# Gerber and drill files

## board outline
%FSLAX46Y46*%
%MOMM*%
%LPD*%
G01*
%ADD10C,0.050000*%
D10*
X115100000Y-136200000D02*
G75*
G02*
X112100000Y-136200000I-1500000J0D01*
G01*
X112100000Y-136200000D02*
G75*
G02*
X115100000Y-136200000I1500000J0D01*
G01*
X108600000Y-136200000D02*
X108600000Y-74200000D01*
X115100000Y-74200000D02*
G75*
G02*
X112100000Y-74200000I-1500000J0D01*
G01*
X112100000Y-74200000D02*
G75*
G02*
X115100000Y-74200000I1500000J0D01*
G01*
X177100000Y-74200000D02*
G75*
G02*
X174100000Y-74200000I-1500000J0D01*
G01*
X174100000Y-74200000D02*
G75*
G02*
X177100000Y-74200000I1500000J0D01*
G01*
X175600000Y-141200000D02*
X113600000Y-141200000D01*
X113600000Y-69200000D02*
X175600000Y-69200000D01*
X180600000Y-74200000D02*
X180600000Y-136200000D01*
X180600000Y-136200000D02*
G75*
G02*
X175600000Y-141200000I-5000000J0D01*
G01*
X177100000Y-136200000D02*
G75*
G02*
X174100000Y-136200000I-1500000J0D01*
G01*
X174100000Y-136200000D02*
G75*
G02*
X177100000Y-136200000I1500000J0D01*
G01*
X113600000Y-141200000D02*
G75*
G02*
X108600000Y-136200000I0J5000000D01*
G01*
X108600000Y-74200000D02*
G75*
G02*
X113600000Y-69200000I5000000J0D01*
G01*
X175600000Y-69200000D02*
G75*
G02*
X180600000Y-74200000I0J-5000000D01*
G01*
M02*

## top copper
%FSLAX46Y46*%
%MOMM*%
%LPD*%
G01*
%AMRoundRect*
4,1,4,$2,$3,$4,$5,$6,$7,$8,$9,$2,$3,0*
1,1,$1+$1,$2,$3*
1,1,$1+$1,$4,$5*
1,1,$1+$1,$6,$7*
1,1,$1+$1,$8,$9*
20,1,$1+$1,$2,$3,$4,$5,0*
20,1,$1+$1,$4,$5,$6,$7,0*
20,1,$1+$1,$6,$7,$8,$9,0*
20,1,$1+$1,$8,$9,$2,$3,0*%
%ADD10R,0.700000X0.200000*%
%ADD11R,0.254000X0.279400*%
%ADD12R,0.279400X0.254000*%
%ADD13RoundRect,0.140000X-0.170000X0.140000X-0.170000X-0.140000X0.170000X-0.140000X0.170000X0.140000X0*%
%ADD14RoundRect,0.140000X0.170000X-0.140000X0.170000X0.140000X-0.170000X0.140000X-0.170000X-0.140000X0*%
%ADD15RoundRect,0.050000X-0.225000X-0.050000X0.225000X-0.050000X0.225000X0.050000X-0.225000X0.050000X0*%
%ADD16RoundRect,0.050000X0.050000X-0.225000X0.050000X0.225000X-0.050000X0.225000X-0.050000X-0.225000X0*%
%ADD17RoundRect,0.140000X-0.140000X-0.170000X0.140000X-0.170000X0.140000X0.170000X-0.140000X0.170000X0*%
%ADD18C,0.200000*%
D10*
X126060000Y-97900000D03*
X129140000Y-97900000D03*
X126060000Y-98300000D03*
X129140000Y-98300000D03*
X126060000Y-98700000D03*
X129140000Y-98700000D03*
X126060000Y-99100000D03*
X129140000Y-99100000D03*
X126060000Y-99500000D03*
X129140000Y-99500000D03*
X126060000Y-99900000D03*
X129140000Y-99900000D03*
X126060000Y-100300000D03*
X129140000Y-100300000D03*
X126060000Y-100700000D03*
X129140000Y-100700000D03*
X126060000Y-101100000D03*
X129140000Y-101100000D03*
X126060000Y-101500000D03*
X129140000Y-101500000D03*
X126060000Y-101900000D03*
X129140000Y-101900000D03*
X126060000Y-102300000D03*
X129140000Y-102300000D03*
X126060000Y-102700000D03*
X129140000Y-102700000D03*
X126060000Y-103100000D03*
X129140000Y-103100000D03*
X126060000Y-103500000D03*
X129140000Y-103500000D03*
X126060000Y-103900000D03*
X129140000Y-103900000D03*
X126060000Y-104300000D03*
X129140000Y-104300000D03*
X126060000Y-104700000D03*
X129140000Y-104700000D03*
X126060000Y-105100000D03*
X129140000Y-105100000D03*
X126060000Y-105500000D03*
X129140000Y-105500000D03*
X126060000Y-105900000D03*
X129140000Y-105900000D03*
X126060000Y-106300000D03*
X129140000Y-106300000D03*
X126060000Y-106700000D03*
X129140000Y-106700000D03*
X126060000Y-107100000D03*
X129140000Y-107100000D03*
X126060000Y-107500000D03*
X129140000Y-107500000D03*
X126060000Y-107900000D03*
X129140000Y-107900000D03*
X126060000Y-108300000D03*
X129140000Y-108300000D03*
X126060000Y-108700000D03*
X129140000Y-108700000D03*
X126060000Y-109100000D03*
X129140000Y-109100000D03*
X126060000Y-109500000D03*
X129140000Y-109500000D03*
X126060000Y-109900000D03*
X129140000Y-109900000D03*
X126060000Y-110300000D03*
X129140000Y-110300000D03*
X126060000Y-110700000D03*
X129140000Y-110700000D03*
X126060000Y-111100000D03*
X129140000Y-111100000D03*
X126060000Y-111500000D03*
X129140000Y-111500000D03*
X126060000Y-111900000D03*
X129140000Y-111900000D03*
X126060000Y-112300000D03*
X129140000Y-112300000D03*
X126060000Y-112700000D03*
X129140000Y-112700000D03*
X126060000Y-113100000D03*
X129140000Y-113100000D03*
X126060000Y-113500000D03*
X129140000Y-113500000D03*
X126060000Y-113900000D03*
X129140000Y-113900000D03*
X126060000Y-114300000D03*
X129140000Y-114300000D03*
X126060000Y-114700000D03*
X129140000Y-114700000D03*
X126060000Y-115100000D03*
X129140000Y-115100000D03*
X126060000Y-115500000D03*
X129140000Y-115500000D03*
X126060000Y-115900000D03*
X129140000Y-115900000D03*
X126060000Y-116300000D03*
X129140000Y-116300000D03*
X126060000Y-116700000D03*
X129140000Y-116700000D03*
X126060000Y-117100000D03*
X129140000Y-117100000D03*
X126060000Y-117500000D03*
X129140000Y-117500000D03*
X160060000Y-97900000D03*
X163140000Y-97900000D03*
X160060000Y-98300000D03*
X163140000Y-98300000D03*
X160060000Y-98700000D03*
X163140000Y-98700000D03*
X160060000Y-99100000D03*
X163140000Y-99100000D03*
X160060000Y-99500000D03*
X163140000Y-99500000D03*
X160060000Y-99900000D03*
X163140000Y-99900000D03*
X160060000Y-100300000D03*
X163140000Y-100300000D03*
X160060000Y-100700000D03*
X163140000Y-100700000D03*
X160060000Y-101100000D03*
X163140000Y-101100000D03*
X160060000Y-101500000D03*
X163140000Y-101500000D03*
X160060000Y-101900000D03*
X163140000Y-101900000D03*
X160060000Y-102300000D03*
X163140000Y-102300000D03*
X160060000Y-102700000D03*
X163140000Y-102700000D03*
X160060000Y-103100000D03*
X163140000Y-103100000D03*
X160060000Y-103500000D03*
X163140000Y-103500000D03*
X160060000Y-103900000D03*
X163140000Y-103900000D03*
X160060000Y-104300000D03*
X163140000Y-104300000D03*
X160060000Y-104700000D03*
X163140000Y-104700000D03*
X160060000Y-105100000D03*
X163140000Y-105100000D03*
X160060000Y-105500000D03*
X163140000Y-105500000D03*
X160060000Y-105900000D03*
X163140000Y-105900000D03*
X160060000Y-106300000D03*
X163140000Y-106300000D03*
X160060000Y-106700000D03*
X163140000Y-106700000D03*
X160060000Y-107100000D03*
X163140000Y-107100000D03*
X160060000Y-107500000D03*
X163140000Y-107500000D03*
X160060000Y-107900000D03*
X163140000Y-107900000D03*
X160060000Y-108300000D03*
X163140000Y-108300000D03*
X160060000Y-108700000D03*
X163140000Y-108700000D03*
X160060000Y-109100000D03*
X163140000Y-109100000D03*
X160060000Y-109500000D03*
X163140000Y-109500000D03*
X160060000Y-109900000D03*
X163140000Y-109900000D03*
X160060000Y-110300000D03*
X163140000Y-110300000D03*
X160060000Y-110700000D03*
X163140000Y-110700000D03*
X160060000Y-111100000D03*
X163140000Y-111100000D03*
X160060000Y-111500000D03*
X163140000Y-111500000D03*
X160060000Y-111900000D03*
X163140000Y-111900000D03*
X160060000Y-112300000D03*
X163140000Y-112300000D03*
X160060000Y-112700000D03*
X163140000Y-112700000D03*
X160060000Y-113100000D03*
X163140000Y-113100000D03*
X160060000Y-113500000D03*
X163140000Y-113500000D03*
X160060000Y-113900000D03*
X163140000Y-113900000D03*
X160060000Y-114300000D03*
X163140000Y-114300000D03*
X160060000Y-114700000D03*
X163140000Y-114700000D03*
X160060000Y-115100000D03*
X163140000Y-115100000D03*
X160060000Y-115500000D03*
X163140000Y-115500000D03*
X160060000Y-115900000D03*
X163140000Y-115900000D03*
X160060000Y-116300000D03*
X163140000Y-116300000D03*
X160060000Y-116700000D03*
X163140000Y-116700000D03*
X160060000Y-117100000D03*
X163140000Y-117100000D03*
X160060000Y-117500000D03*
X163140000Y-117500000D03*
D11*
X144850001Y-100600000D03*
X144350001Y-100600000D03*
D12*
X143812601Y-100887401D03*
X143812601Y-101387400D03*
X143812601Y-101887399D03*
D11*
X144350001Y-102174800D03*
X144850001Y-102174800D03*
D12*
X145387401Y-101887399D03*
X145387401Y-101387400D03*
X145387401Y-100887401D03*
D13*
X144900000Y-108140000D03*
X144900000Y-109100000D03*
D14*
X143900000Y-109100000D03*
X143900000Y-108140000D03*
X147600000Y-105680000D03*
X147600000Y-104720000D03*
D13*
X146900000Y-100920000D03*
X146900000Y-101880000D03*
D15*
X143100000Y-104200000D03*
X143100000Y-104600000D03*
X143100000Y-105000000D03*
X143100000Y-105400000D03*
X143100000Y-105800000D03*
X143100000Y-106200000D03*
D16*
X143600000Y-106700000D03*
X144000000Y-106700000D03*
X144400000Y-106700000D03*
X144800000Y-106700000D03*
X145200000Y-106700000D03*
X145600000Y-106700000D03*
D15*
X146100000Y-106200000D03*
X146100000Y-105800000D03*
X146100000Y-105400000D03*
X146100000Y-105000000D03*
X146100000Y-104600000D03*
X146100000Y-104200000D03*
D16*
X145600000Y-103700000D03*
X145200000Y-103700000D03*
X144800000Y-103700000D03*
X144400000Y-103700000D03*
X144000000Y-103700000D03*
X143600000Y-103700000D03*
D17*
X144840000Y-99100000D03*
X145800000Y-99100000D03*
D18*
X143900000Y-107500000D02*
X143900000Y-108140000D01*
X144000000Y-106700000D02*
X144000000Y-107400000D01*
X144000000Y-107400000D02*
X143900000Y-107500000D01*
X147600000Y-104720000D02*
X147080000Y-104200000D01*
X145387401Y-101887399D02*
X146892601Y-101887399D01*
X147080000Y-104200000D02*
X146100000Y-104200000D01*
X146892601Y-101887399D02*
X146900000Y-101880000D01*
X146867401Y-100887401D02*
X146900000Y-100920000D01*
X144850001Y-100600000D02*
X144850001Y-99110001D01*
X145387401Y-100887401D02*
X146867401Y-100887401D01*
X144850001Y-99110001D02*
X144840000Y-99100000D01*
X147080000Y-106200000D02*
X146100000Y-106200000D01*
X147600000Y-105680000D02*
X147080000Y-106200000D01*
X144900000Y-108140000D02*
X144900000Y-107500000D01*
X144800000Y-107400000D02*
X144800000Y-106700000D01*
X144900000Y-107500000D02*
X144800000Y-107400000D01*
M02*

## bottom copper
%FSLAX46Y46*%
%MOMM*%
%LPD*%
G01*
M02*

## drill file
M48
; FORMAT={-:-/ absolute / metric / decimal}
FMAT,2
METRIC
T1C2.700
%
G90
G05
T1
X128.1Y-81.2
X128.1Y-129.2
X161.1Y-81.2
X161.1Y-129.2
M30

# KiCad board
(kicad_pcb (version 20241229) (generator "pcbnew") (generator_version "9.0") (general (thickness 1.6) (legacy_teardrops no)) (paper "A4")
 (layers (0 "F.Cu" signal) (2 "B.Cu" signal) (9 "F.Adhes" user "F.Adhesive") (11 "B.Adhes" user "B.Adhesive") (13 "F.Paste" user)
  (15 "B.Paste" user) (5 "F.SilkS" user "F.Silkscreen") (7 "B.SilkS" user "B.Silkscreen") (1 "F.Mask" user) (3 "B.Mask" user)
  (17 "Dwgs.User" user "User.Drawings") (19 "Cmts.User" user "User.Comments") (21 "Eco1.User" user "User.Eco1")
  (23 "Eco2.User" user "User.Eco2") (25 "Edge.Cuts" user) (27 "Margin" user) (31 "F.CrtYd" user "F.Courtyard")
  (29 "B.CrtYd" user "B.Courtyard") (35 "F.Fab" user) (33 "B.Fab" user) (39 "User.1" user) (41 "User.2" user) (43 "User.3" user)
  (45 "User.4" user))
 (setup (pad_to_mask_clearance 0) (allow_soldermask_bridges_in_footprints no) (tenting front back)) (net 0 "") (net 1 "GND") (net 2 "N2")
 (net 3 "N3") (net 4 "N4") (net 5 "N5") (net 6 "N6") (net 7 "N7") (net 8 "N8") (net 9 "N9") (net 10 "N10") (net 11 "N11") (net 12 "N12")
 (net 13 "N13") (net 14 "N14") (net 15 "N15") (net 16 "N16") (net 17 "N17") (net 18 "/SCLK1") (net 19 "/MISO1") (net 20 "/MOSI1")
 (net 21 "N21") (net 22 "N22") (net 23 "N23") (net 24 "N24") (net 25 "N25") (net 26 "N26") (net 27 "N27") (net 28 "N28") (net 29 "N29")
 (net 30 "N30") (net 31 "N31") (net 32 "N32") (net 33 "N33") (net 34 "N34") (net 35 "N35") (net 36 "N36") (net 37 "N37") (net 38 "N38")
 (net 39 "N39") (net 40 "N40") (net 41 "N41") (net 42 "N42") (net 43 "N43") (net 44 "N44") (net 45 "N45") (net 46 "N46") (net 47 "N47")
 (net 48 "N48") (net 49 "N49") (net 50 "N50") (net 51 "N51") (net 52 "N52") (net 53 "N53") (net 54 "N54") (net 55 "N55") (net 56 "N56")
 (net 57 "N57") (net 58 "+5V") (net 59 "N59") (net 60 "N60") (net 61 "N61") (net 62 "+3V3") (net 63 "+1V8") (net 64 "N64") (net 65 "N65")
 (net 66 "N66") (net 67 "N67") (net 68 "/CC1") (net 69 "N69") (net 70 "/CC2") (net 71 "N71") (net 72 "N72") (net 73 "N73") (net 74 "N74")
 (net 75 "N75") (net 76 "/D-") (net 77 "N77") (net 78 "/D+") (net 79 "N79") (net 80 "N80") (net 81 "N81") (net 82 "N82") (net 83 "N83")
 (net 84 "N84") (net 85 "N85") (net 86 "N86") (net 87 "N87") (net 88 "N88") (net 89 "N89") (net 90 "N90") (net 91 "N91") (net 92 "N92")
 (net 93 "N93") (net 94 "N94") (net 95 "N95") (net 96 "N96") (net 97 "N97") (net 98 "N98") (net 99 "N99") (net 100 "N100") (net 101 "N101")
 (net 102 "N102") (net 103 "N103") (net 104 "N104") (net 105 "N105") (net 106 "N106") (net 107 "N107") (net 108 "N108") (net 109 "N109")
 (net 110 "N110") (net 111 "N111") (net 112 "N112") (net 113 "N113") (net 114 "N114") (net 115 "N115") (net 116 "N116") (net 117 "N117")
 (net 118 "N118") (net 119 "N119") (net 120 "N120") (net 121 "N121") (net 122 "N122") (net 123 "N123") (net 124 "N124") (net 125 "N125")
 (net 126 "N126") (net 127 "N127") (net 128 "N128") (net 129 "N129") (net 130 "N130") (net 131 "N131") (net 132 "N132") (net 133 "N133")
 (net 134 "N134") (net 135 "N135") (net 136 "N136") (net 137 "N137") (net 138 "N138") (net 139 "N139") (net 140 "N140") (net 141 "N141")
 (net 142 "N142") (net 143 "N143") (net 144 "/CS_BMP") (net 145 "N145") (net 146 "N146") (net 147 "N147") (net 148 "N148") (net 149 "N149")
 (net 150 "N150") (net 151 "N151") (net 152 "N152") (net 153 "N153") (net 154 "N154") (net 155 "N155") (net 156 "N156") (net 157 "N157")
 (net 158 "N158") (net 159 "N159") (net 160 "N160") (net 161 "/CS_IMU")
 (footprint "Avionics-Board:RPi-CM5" (layer "F.Cu") (at 128.1 129.2)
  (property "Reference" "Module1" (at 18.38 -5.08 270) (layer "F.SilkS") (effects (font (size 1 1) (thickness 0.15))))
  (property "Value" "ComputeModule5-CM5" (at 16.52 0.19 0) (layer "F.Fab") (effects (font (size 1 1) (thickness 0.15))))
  (pad "" np_thru_hole circle (at 0 -48) (size 2.7 2.7) (drill 2.7) (layers "*.Cu" "*.Mask") (solder_mask_margin 1.7) (clearance 1.7))
  (pad "" np_thru_hole circle (at 0 0) (size 2.7 2.7) (drill 2.7) (layers "*.Cu" "*.Mask") (solder_mask_margin 1.7) (clearance 1.7))
  (pad "" np_thru_hole circle (at 33 -48) (size 2.7 2.7) (drill 2.7) (layers "*.Cu" "*.Mask") (solder_mask_margin 1.7) (clearance 1.7))
  (pad "" np_thru_hole circle (at 33 0) (size 2.7 2.7) (drill 2.7) (layers "*.Cu" "*.Mask") (solder_mask_margin 1.7) (clearance 1.7))
  (pad "1" smd rect (at -2.04 -31.3 270) (size 0.2 0.7) (layers "F.Cu" "F.Mask" "F.Paste") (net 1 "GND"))
  (pad "2" smd rect (at 1.04 -31.3 270) (size 0.2 0.7) (layers "F.Cu" "F.Mask" "F.Paste") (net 1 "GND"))
  (pad "3" smd rect (at -2.04 -30.9 270) (size 0.2 0.7) (layers "F.Cu" "F.Mask" "F.Paste") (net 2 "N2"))
  (pad "4" smd rect (at 1.04 -30.9 270) (size 0.2 0.7) (layers "F.Cu" "F.Mask" "F.Paste") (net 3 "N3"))
  (pad "5" smd rect (at -2.04 -30.5 270) (size 0.2 0.7) (layers "F.Cu" "F.Mask" "F.Paste") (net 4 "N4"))
  (pad "6" smd rect (at 1.04 -30.5 270) (size 0.2 0.7) (layers "F.Cu" "F.Mask" "F.Paste") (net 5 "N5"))
  (pad "7" smd rect (at -2.04 -30.1 270) (size 0.2 0.7) (layers "F.Cu" "F.Mask" "F.Paste") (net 1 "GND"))
  (pad "8" smd rect (at 1.04 -30.1 270) (size 0.2 0.7) (layers "F.Cu" "F.Mask" "F.Paste") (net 1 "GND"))
  (pad "9" smd rect (at -2.04 -29.7 270) (size 0.2 0.7) (layers "F.Cu" "F.Mask" "F.Paste") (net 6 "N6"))
  (pad "10" smd rect (at 1.04 -29.7 270) (size 0.2 0.7) (layers "F.Cu" "F.Mask" "F.Paste") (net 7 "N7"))
  (pad "11" smd rect (at -2.04 -29.3 270) (size 0.2 0.7) (layers "F.Cu" "F.Mask" "F.Paste") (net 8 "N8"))
  (pad "12" smd rect (at 1.04 -29.3 270) (size 0.2 0.7) (layers "F.Cu" "F.Mask" "F.Paste") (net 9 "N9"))
  (pad "13" smd rect (at -2.04 -28.9 270) (size 0.2 0.7) (layers "F.Cu" "F.Mask" "F.Paste") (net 1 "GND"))
  (pad "14" smd rect (at 1.04 -28.9 270) (size 0.2 0.7) (layers "F.Cu" "F.Mask" "F.Paste") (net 1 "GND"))
  (pad "15" smd rect (at -2.04 -28.5 270) (size 0.2 0.7) (layers "F.Cu" "F.Mask" "F.Paste") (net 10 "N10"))
  (pad "16" smd rect (at 1.04 -28.5 270) (size 0.2 0.7) (layers "F.Cu" "F.Mask" "F.Paste") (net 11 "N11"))
  (pad "17" smd rect (at -2.04 -28.1 270) (size 0.2 0.7) (layers "F.Cu" "F.Mask" "F.Paste") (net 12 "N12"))
  (pad "18" smd rect (at 1.04 -28.1 270) (size 0.2 0.7) (layers "F.Cu" "F.Mask" "F.Paste") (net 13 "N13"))
  (pad "19" smd rect (at -2.04 -27.7 270) (size 0.2 0.7) (layers "F.Cu" "F.Mask" "F.Paste") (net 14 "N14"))
  (pad "20" smd rect (at 1.04 -27.7 270) (size 0.2 0.7) (layers "F.Cu" "F.Mask" "F.Paste") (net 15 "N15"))
  (pad "21" smd rect (at -2.04 -27.3 270) (size 0.2 0.7) (layers "F.Cu" "F.Mask" "F.Paste") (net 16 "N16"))
  (pad "22" smd rect (at 1.04 -27.3 270) (size 0.2 0.7) (layers "F.Cu" "F.Mask" "F.Paste") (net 1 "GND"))
  (pad "23" smd rect (at -2.04 -26.9 270) (size 0.2 0.7) (layers "F.Cu" "F.Mask" "F.Paste") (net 1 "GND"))
  (pad "24" smd rect (at 1.04 -26.9 270) (size 0.2 0.7) (layers "F.Cu" "F.Mask" "F.Paste") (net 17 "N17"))
  (pad "25" smd rect (at -2.04 -26.5 270) (size 0.2 0.7) (layers "F.Cu" "F.Mask" "F.Paste") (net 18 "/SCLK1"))
  (pad "26" smd rect (at 1.04 -26.5 270) (size 0.2 0.7) (layers "F.Cu" "F.Mask" "F.Paste") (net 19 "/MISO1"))
  (pad "27" smd rect (at -2.04 -26.1 270) (size 0.2 0.7) (layers "F.Cu" "F.Mask" "F.Paste") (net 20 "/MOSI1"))
  (pad "28" smd rect (at 1.04 -26.1 270) (size 0.2 0.7) (layers "F.Cu" "F.Mask" "F.Paste") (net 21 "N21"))
  (pad "29" smd rect (at -2.04 -25.7 270) (size 0.2 0.7) (layers "F.Cu" "F.Mask" "F.Paste") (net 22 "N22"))
  (pad "30" smd rect (at 1.04 -25.7 270) (size 0.2 0.7) (layers "F.Cu" "F.Mask" "F.Paste") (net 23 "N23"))
  (pad "31" smd rect (at -2.04 -25.3 270) (size 0.2 0.7) (layers "F.Cu" "F.Mask" "F.Paste") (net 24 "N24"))
  (pad "32" smd rect (at 1.04 -25.3 270) (size 0.2 0.7) (layers "F.Cu" "F.Mask" "F.Paste") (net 1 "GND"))
  (pad "33" smd rect (at -2.04 -24.9 270) (size 0.2 0.7) (layers "F.Cu" "F.Mask" "F.Paste") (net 1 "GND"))
  (pad "34" smd rect (at 1.04 -24.9 270) (size 0.2 0.7) (layers "F.Cu" "F.Mask" "F.Paste") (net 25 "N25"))
  (pad "35" smd rect (at -2.04 -24.5 270) (size 0.2 0.7) (layers "F.Cu" "F.Mask" "F.Paste") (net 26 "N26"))
  (pad "36" smd rect (at 1.04 -24.5 270) (size 0.2 0.7) (layers "F.Cu" "F.Mask" "F.Paste") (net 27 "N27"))
  (pad "37" smd rect (at -2.04 -24.1 270) (size 0.2 0.7) (layers "F.Cu" "F.Mask" "F.Paste") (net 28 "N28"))
  (pad "38" smd rect (at 1.04 -24.1 270) (size 0.2 0.7) (layers "F.Cu" "F.Mask" "F.Paste") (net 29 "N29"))
  (pad "39" smd rect (at -2.04 -23.7 270) (size 0.2 0.7) (layers "F.Cu" "F.Mask" "F.Paste") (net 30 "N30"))
  (pad "40" smd rect (at 1.04 -23.7 270) (size 0.2 0.7) (layers "F.Cu" "F.Mask" "F.Paste") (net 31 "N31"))
  (pad "41" smd rect (at -2.04 -23.3 270) (size 0.2 0.7) (layers "F.Cu" "F.Mask" "F.Paste") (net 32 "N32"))
  (pad "42" smd rect (at 1.04 -23.3 270) (size 0.2 0.7) (layers "F.Cu" "F.Mask" "F.Paste") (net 1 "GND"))
  (pad "43" smd rect (at -2.04 -22.9 270) (size 0.2 0.7) (layers "F.Cu" "F.Mask" "F.Paste") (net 1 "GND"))
  (pad "44" smd rect (at 1.04 -22.9 270) (size 0.2 0.7) (layers "F.Cu" "F.Mask" "F.Paste") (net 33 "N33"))
  (pad "45" smd rect (at -2.04 -22.5 270) (size 0.2 0.7) (layers "F.Cu" "F.Mask" "F.Paste") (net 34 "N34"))
  (pad "46" smd rect (at 1.04 -22.5 270) (size 0.2 0.7) (layers "F.Cu" "F.Mask" "F.Paste") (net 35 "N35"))
  (pad "47" smd rect (at -2.04 -22.1 270) (size 0.2 0.7) (layers "F.Cu" "F.Mask" "F.Paste") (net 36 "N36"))
  (pad "48" smd rect (at 1.04 -22.1 270) (size 0.2 0.7) (layers "F.Cu" "F.Mask" "F.Paste") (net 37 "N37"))
  (pad "49" smd rect (at -2.04 -21.7 270) (size 0.2 0.7) (layers "F.Cu" "F.Mask" "F.Paste") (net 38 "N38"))
  (pad "50" smd rect (at 1.04 -21.7 270) (size 0.2 0.7) (layers "F.Cu" "F.Mask" "F.Paste") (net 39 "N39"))
  (pad "51" smd rect (at -2.04 -21.3 270) (size 0.2 0.7) (layers "F.Cu" "F.Mask" "F.Paste") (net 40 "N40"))
  (pad "52" smd rect (at 1.04 -21.3 270) (size 0.2 0.7) (layers "F.Cu" "F.Mask" "F.Paste") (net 1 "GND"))
  (pad "53" smd rect (at -2.04 -20.9 270) (size 0.2 0.7) (layers "F.Cu" "F.Mask" "F.Paste") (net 1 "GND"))
  (pad "54" smd rect (at 1.04 -20.9 270) (size 0.2 0.7) (layers "F.Cu" "F.Mask" "F.Paste") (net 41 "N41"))
  (pad "55" smd rect (at -2.04 -20.5 270) (size 0.2 0.7) (layers "F.Cu" "F.Mask" "F.Paste") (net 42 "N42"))
  (pad "56" smd rect (at 1.04 -20.5 270) (size 0.2 0.7) (layers "F.Cu" "F.Mask" "F.Paste") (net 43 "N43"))
  (pad "57" smd rect (at -2.04 -20.1 270) (size 0.2 0.7) (layers "F.Cu" "F.Mask" "F.Paste") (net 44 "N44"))
  (pad "58" smd rect (at 1.04 -20.1 270) (size 0.2 0.7) (layers "F.Cu" "F.Mask" "F.Paste") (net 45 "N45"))
  (pad "59" smd rect (at -2.04 -19.7 270) (size 0.2 0.7) (layers "F.Cu" "F.Mask" "F.Paste") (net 1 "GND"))
  (pad "60" smd rect (at 1.04 -19.7 270) (size 0.2 0.7) (layers "F.Cu" "F.Mask" "F.Paste") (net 1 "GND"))
  (pad "61" smd rect (at -2.04 -19.3 270) (size 0.2 0.7) (layers "F.Cu" "F.Mask" "F.Paste") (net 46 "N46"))
  (pad "62" smd rect (at 1.04 -19.3 270) (size 0.2 0.7) (layers "F.Cu" "F.Mask" "F.Paste") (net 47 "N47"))
  (pad "63" smd rect (at -2.04 -18.9 270) (size 0.2 0.7) (layers "F.Cu" "F.Mask" "F.Paste") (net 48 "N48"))
  (pad "64" smd rect (at 1.04 -18.9 270) (size 0.2 0.7) (layers "F.Cu" "F.Mask" "F.Paste") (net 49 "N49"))
  (pad "65" smd rect (at -2.04 -18.5 270) (size 0.2 0.7) (layers "F.Cu" "F.Mask" "F.Paste") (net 1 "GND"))
  (pad "66" smd rect (at 1.04 -18.5 270) (size 0.2 0.7) (layers "F.Cu" "F.Mask" "F.Paste") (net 1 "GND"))
  (pad "67" smd rect (at -2.04 -18.1 270) (size 0.2 0.7) (layers "F.Cu" "F.Mask" "F.Paste") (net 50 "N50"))
  (pad "68" smd rect (at 1.04 -18.1 270) (size 0.2 0.7) (layers "F.Cu" "F.Mask" "F.Paste") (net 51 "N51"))
  (pad "69" smd rect (at -2.04 -17.7 270) (size 0.2 0.7) (layers "F.Cu" "F.Mask" "F.Paste") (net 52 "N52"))
  (pad "70" smd rect (at 1.04 -17.7 270) (size 0.2 0.7) (layers "F.Cu" "F.Mask" "F.Paste") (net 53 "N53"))
  (pad "71" smd rect (at -2.04 -17.3 270) (size 0.2 0.7) (layers "F.Cu" "F.Mask" "F.Paste") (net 1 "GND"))
  (pad "72" smd rect (at 1.04 -17.3 270) (size 0.2 0.7) (layers "F.Cu" "F.Mask" "F.Paste") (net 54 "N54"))
  (pad "73" smd rect (at -2.04 -16.9 270) (size 0.2 0.7) (layers "F.Cu" "F.Mask" "F.Paste") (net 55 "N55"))
  (pad "74" smd rect (at 1.04 -16.9 270) (size 0.2 0.7) (layers "F.Cu" "F.Mask" "F.Paste") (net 1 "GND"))
  (pad "75" smd rect (at -2.04 -16.5 270) (size 0.2 0.7) (layers "F.Cu" "F.Mask" "F.Paste") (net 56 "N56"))
  (pad "76" smd rect (at 1.04 -16.5 270) (size 0.2 0.7) (layers "F.Cu" "F.Mask" "F.Paste") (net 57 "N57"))
  (pad "77" smd rect (at -2.04 -16.1 270) (size 0.2 0.7) (layers "F.Cu" "F.Mask" "F.Paste") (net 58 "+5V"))
  (pad "78" smd rect (at 1.04 -16.1 270) (size 0.2 0.7) (layers "F.Cu" "F.Mask" "F.Paste") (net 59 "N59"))
  (pad "79" smd rect (at -2.04 -15.7 270) (size 0.2 0.7) (layers "F.Cu" "F.Mask" "F.Paste") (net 58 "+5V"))
  (pad "80" smd rect (at 1.04 -15.7 270) (size 0.2 0.7) (layers "F.Cu" "F.Mask" "F.Paste") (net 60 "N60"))
  (pad "81" smd rect (at -2.04 -15.3 270) (size 0.2 0.7) (layers "F.Cu" "F.Mask" "F.Paste") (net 58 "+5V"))
  (pad "82" smd rect (at 1.04 -15.3 270) (size 0.2 0.7) (layers "F.Cu" "F.Mask" "F.Paste") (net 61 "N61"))
  (pad "83" smd rect (at -2.04 -14.9 270) (size 0.2 0.7) (layers "F.Cu" "F.Mask" "F.Paste") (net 58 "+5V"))
  (pad "84" smd rect (at 1.04 -14.9 270) (size 0.2 0.7) (layers "F.Cu" "F.Mask" "F.Paste") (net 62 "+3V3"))
  (pad "85" smd rect (at -2.04 -14.5 270) (size 0.2 0.7) (layers "F.Cu" "F.Mask" "F.Paste") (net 58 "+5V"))
  (pad "86" smd rect (at 1.04 -14.5 270) (size 0.2 0.7) (layers "F.Cu" "F.Mask" "F.Paste") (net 62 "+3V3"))
  (pad "87" smd rect (at -2.04 -14.1 270) (size 0.2 0.7) (layers "F.Cu" "F.Mask" "F.Paste") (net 58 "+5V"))
  (pad "88" smd rect (at 1.04 -14.1 270) (size 0.2 0.7) (layers "F.Cu" "F.Mask" "F.Paste") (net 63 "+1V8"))
  (pad "89" smd rect (at -2.04 -13.7 270) (size 0.2 0.7) (layers "F.Cu" "F.Mask" "F.Paste") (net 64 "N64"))
  (pad "90" smd rect (at 1.04 -13.7 270) (size 0.2 0.7) (layers "F.Cu" "F.Mask" "F.Paste") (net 63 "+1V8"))
  (pad "91" smd rect (at -2.04 -13.3 270) (size 0.2 0.7) (layers "F.Cu" "F.Mask" "F.Paste") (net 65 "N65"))
  (pad "92" smd rect (at 1.04 -13.3 270) (size 0.2 0.7) (layers "F.Cu" "F.Mask" "F.Paste") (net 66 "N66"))
  (pad "93" smd rect (at -2.04 -12.9 270) (size 0.2 0.7) (layers "F.Cu" "F.Mask" "F.Paste") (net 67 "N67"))
  (pad "94" smd rect (at 1.04 -12.9 270) (size 0.2 0.7) (layers "F.Cu" "F.Mask" "F.Paste") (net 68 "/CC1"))
  (pad "95" smd rect (at -2.04 -12.5 270) (size 0.2 0.7) (layers "F.Cu" "F.Mask" "F.Paste") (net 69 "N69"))
  (pad "96" smd rect (at 1.04 -12.5 270) (size 0.2 0.7) (layers "F.Cu" "F.Mask" "F.Paste") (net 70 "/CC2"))
  (pad "97" smd rect (at -2.04 -12.1 270) (size 0.2 0.7) (layers "F.Cu" "F.Mask" "F.Paste") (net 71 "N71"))
  (pad "98" smd rect (at 1.04 -12.1 270) (size 0.2 0.7) (layers "F.Cu" "F.Mask" "F.Paste") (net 1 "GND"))
  (pad "99" smd rect (at -2.04 -11.7 270) (size 0.2 0.7) (layers "F.Cu" "F.Mask" "F.Paste") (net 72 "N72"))
  (pad "100" smd rect (at 1.04 -11.7 270) (size 0.2 0.7) (layers "F.Cu" "F.Mask" "F.Paste") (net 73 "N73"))
  (pad "101" smd rect (at 31.96 -31.3 270) (size 0.2 0.7) (layers "F.Cu" "F.Mask" "F.Paste") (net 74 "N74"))
  (pad "102" smd rect (at 35.04 -31.3 270) (size 0.2 0.7) (layers "F.Cu" "F.Mask" "F.Paste") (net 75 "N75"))
  (pad "103" smd rect (at 31.96 -30.9 270) (size 0.2 0.7) (layers "F.Cu" "F.Mask" "F.Paste") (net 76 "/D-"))
  (pad "104" smd rect (at 35.04 -30.9 270) (size 0.2 0.7) (layers "F.Cu" "F.Mask" "F.Paste") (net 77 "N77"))
  (pad "105" smd rect (at 31.96 -30.5 270) (size 0.2 0.7) (layers "F.Cu" "F.Mask" "F.Paste") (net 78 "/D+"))
  (pad "106" smd rect (at 35.04 -30.5 270) (size 0.2 0.7) (layers "F.Cu" "F.Mask" "F.Paste") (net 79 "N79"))
  (pad "107" smd rect (at 31.96 -30.1 270) (size 0.2 0.7) (layers "F.Cu" "F.Mask" "F.Paste") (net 1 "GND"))
  (pad "108" smd rect (at 35.04 -30.1 270) (size 0.2 0.7) (layers "F.Cu" "F.Mask" "F.Paste") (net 1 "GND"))
  (pad "109" smd rect (at 31.96 -29.7 270) (size 0.2 0.7) (layers "F.Cu" "F.Mask" "F.Paste") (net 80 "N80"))
  (pad "110" smd rect (at 35.04 -29.7 270) (size 0.2 0.7) (layers "F.Cu" "F.Mask" "F.Paste") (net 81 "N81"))
  (pad "111" smd rect (at 31.96 -29.3 270) (size 0.2 0.7) (layers "F.Cu" "F.Mask" "F.Paste") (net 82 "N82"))
  (pad "112" smd rect (at 35.04 -29.3 270) (size 0.2 0.7) (layers "F.Cu" "F.Mask" "F.Paste") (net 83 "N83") (die_length 0.01))
  (pad "113" smd rect (at 31.96 -28.9 270) (size 0.2 0.7) (layers "F.Cu" "F.Mask" "F.Paste") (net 1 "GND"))
  (pad "114" smd rect (at 35.04 -28.9 270) (size 0.2 0.7) (layers "F.Cu" "F.Mask" "F.Paste") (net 1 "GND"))
  (pad "115" smd rect (at 31.96 -28.5 270) (size 0.2 0.7) (layers "F.Cu" "F.Mask" "F.Paste") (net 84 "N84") (die_length 0.01))
  (pad "116" smd rect (at 35.04 -28.5 270) (size 0.2 0.7) (layers "F.Cu" "F.Mask" "F.Paste") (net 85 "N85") (die_length 0.84))
  (pad "117" smd rect (at 31.96 -28.1 270) (size 0.2 0.7) (layers "F.Cu" "F.Mask" "F.Paste") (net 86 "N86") (die_length 0.02))
  (pad "118" smd rect (at 35.04 -28.1 270) (size 0.2 0.7) (layers "F.Cu" "F.Mask" "F.Paste") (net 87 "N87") (die_length 0.84))
  (pad "119" smd rect (at 31.96 -27.7 270) (size 0.2 0.7) (layers "F.Cu" "F.Mask" "F.Paste") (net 1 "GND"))
  (pad "120" smd rect (at 35.04 -27.7 270) (size 0.2 0.7) (layers "F.Cu" "F.Mask" "F.Paste") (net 1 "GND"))
  (pad "121" smd rect (at 31.96 -27.3 270) (size 0.2 0.7) (layers "F.Cu" "F.Mask" "F.Paste") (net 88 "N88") (die_length 0.4))
  (pad "122" smd rect (at 35.04 -27.3 270) (size 0.2 0.7) (layers "F.Cu" "F.Mask" "F.Paste") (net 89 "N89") (die_length 3.71))
  (pad "123" smd rect (at 31.96 -26.9 270) (size 0.2 0.7) (layers "F.Cu" "F.Mask" "F.Paste") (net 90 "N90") (die_length 0.4))
  (pad "124" smd rect (at 35.04 -26.9 270) (size 0.2 0.7) (layers "F.Cu" "F.Mask" "F.Paste") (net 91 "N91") (die_length 3.72))
  (pad "125" smd rect (at 31.96 -26.5 270) (size 0.2 0.7) (layers "F.Cu" "F.Mask" "F.Paste") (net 1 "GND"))
  (pad "126" smd rect (at 35.04 -26.5 270) (size 0.2 0.7) (layers "F.Cu" "F.Mask" "F.Paste") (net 1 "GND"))
  (pad "127" smd rect (at 31.96 -26.1 270) (size 0.2 0.7) (layers "F.Cu" "F.Mask" "F.Paste") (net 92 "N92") (die_length 0.78))
  (pad "128" smd rect (at 35.04 -26.1 270) (size 0.2 0.7) (layers "F.Cu" "F.Mask" "F.Paste") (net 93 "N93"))
  (pad "129" smd rect (at 31.96 -25.7 270) (size 0.2 0.7) (layers "F.Cu" "F.Mask" "F.Paste") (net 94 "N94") (die_length 0.78))
  (pad "130" smd rect (at 35.04 -25.7 270) (size 0.2 0.7) (layers "F.Cu" "F.Mask" "F.Paste") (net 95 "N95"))
  (pad "131" smd rect (at 31.96 -25.3 270) (size 0.2 0.7) (layers "F.Cu" "F.Mask" "F.Paste") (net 1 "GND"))
  (pad "132" smd rect (at 35.04 -25.3 270) (size 0.2 0.7) (layers "F.Cu" "F.Mask" "F.Paste") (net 1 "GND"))
  (pad "133" smd rect (at 31.96 -24.9 270) (size 0.2 0.7) (layers "F.Cu" "F.Mask" "F.Paste") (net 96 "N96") (die_length 0.04))
  (pad "134" smd rect (at 35.04 -24.9 270) (size 0.2 0.7) (layers "F.Cu" "F.Mask" "F.Paste") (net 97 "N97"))
  (pad "135" smd rect (at 31.96 -24.5 270) (size 0.2 0.7) (layers "F.Cu" "F.Mask" "F.Paste") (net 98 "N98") (die_length 0.03))
  (pad "136" smd rect (at 35.04 -24.5 270) (size 0.2 0.7) (layers "F.Cu" "F.Mask" "F.Paste") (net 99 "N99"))
  (pad "137" smd rect (at 31.96 -24.1 270) (size 0.2 0.7) (layers "F.Cu" "F.Mask" "F.Paste") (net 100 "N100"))
  (pad "138" smd rect (at 35.04 -24.1 270) (size 0.2 0.7) (layers "F.Cu" "F.Mask" "F.Paste") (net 1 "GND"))
  (pad "139" smd rect (at 31.96 -23.7 270) (size 0.2 0.7) (layers "F.Cu" "F.Mask" "F.Paste") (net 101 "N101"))
  (pad "140" smd rect (at 35.04 -23.7 270) (size 0.2 0.7) (layers "F.Cu" "F.Mask" "F.Paste") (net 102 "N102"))
  (pad "141" smd rect (at 31.96 -23.3 270) (size 0.2 0.7) (layers "F.Cu" "F.Mask" "F.Paste") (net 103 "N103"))
  (pad "142" smd rect (at 35.04 -23.3 270) (size 0.2 0.7) (layers "F.Cu" "F.Mask" "F.Paste") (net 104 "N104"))
  (pad "143" smd rect (at 31.96 -22.9 270) (size 0.2 0.7) (layers "F.Cu" "F.Mask" "F.Paste") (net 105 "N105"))
  (pad "144" smd rect (at 35.04 -22.9 270) (size 0.2 0.7) (layers "F.Cu" "F.Mask" "F.Paste") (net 1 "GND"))
  (pad "145" smd rect (at 31.96 -22.5 270) (size 0.2 0.7) (layers "F.Cu" "F.Mask" "F.Paste") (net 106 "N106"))
  (pad "146" smd rect (at 35.04 -22.5 270) (size 0.2 0.7) (layers "F.Cu" "F.Mask" "F.Paste") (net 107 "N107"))
  (pad "147" smd rect (at 31.96 -22.1 270) (size 0.2 0.7) (layers "F.Cu" "F.Mask" "F.Paste") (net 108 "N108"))
  (pad "148" smd rect (at 35.04 -22.1 270) (size 0.2 0.7) (layers "F.Cu" "F.Mask" "F.Paste") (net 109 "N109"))
  (pad "149" smd rect (at 31.96 -21.7 270) (size 0.2 0.7) (layers "F.Cu" "F.Mask" "F.Paste") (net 1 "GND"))
  (pad "150" smd rect (at 35.04 -21.7 270) (size 0.2 0.7) (layers "F.Cu" "F.Mask" "F.Paste") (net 1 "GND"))
  (pad "151" smd rect (at 31.96 -21.3 270) (size 0.2 0.7) (layers "F.Cu" "F.Mask" "F.Paste") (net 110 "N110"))
  (pad "152" smd rect (at 35.04 -21.3 270) (size 0.2 0.7) (layers "F.Cu" "F.Mask" "F.Paste") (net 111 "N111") (die_length 5.18))
  (pad "153" smd rect (at 31.96 -20.9 270) (size 0.2 0.7) (layers "F.Cu" "F.Mask" "F.Paste") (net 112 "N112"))
  (pad "154" smd rect (at 35.04 -20.9 270) (size 0.2 0.7) (layers "F.Cu" "F.Mask" "F.Paste") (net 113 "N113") (die_length 5.18))
  (pad "155" smd rect (at 31.96 -20.5 270) (size 0.2 0.7) (layers "F.Cu" "F.Mask" "F.Paste") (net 1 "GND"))
  (pad "156" smd rect (at 35.04 -20.5 270) (size 0.2 0.7) (layers "F.Cu" "F.Mask" "F.Paste") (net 1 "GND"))
  (pad "157" smd rect (at 31.96 -20.1 270) (size 0.2 0.7) (layers "F.Cu" "F.Mask" "F.Paste") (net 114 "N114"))
  (pad "158" smd rect (at 35.04 -20.1 270) (size 0.2 0.7) (layers "F.Cu" "F.Mask" "F.Paste") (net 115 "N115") (die_length 4.75))
  (pad "159" smd rect (at 31.96 -19.7 270) (size 0.2 0.7) (layers "F.Cu" "F.Mask" "F.Paste") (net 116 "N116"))
  (pad "160" smd rect (at 35.04 -19.7 270) (size 0.2 0.7) (layers "F.Cu" "F.Mask" "F.Paste") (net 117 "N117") (die_length 4.76))
  (pad "161" smd rect (at 31.96 -19.3 270) (size 0.2 0.7) (layers "F.Cu" "F.Mask" "F.Paste") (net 1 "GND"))
  (pad "162" smd rect (at 35.04 -19.3 270) (size 0.2 0.7) (layers "F.Cu" "F.Mask" "F.Paste") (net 1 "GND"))
  (pad "163" smd rect (at 31.96 -18.9 270) (size 0.2 0.7) (layers "F.Cu" "F.Mask" "F.Paste") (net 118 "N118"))
  (pad "164" smd rect (at 35.04 -18.9 270) (size 0.2 0.7) (layers "F.Cu" "F.Mask" "F.Paste") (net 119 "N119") (die_length 2.99))
  (pad "165" smd rect (at 31.96 -18.5 270) (size 0.2 0.7) (layers "F.Cu" "F.Mask" "F.Paste") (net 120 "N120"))
  (pad "166" smd rect (at 35.04 -18.5 270) (size 0.2 0.7) (layers "F.Cu" "F.Mask" "F.Paste") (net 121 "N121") (die_length 2.99))
  (pad "167" smd rect (at 31.96 -18.1 270) (size 0.2 0.7) (layers "F.Cu" "F.Mask" "F.Paste") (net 1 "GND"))
  (pad "168" smd rect (at 35.04 -18.1 270) (size 0.2 0.7) (layers "F.Cu" "F.Mask" "F.Paste") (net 1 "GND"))
  (pad "169" smd rect (at 31.96 -17.7 270) (size 0.2 0.7) (layers "F.Cu" "F.Mask" "F.Paste") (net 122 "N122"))
  (pad "170" smd rect (at 35.04 -17.7 270) (size 0.2 0.7) (layers "F.Cu" "F.Mask" "F.Paste") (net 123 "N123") (die_length 0.25))
  (pad "171" smd rect (at 31.96 -17.3 270) (size 0.2 0.7) (layers "F.Cu" "F.Mask" "F.Paste") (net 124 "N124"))
  (pad "172" smd rect (at 35.04 -17.3 270) (size 0.2 0.7) (layers "F.Cu" "F.Mask" "F.Paste") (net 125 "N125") (die_length 0.25))
  (pad "173" smd rect (at 31.96 -16.9 270) (size 0.2 0.7) (layers "F.Cu" "F.Mask" "F.Paste") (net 1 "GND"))
  (pad "174" smd rect (at 35.04 -16.9 270) (size 0.2 0.7) (layers "F.Cu" "F.Mask" "F.Paste") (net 1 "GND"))
  (pad "175" smd rect (at 31.96 -16.5 270) (size 0.2 0.7) (layers "F.Cu" "F.Mask" "F.Paste") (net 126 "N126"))
  (pad "176" smd rect (at 35.04 -16.5 270) (size 0.2 0.7) (layers "F.Cu" "F.Mask" "F.Paste") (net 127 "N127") (die_length 5.18))
  (pad "177" smd rect (at 31.96 -16.1 270) (size 0.2 0.7) (layers "F.Cu" "F.Mask" "F.Paste") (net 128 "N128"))
  (pad "178" smd rect (at 35.04 -16.1 270) (size 0.2 0.7) (layers "F.Cu" "F.Mask" "F.Paste") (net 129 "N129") (die_length 5.18))
  (pad "179" smd rect (at 31.96 -15.7 270) (size 0.2 0.7) (layers "F.Cu" "F.Mask" "F.Paste") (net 1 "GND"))
  (pad "180" smd rect (at 35.04 -15.7 270) (size 0.2 0.7) (layers "F.Cu" "F.Mask" "F.Paste") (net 1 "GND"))
  (pad "181" smd rect (at 31.96 -15.3 270) (size 0.2 0.7) (layers "F.Cu" "F.Mask" "F.Paste") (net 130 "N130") (die_length 1.06))
  (pad "182" smd rect (at 35.04 -15.3 270) (size 0.2 0.7) (layers "F.Cu" "F.Mask" "F.Paste") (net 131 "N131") (die_length 0.18))
  (pad "183" smd rect (at 31.96 -14.9 270) (size 0.2 0.7) (layers "F.Cu" "F.Mask" "F.Paste") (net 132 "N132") (die_length 1.05))
  (pad "184" smd rect (at 35.04 -14.9 270) (size 0.2 0.7) (layers "F.Cu" "F.Mask" "F.Paste") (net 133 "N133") (die_length 0.18))
  (pad "185" smd rect (at 31.96 -14.5 270) (size 0.2 0.7) (layers "F.Cu" "F.Mask" "F.Paste") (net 1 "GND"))
  (pad "186" smd rect (at 35.04 -14.5 270) (size 0.2 0.7) (layers "F.Cu" "F.Mask" "F.Paste") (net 1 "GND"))
  (pad "187" smd rect (at 31.96 -14.1 270) (size 0.2 0.7) (layers "F.Cu" "F.Mask" "F.Paste") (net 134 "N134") (die_length 1.28))
  (pad "188" smd rect (at 35.04 -14.1 270) (size 0.2 0.7) (layers "F.Cu" "F.Mask" "F.Paste") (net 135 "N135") (die_length 0.91))
  (pad "189" smd rect (at 31.96 -13.7 270) (size 0.2 0.7) (layers "F.Cu" "F.Mask" "F.Paste") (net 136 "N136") (die_length 1.27))
  (pad "190" smd rect (at 35.04 -13.7 270) (size 0.2 0.7) (layers "F.Cu" "F.Mask" "F.Paste") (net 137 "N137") (die_length 0.91))
  (pad "191" smd rect (at 31.96 -13.3 270) (size 0.2 0.7) (layers "F.Cu" "F.Mask" "F.Paste") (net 1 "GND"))
  (pad "192" smd rect (at 35.04 -13.3 270) (size 0.2 0.7) (layers "F.Cu" "F.Mask" "F.Paste") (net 1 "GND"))
  (pad "193" smd rect (at 31.96 -12.9 270) (size 0.2 0.7) (layers "F.Cu" "F.Mask" "F.Paste") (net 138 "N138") (die_length 0.83))
  (pad "194" smd rect (at 35.04 -12.9 270) (size 0.2 0.7) (layers "F.Cu" "F.Mask" "F.Paste") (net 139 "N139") (die_length 3.79))
  (pad "195" smd rect (at 31.96 -12.5 270) (size 0.2 0.7) (layers "F.Cu" "F.Mask" "F.Paste") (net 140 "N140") (die_length 0.84))
  (pad "196" smd rect (at 35.04 -12.5 270) (size 0.2 0.7) (layers "F.Cu" "F.Mask" "F.Paste") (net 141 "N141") (die_length 3.79))
  (pad "197" smd rect (at 31.96 -12.1 270) (size 0.2 0.7) (layers "F.Cu" "F.Mask" "F.Paste") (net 1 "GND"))
  (pad "198" smd rect (at 35.04 -12.1 270) (size 0.2 0.7) (layers "F.Cu" "F.Mask" "F.Paste") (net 1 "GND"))
  (pad "199" smd rect (at 31.96 -11.7 270) (size 0.2 0.7) (layers "F.Cu" "F.Mask" "F.Paste") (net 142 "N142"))
  (pad "200" smd rect (at 35.04 -11.7 270) (size 0.2 0.7) (layers "F.Cu" "F.Mask" "F.Paste") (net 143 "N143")))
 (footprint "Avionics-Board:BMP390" (layer "F.Cu") (at 144.600001 101.3874 -90)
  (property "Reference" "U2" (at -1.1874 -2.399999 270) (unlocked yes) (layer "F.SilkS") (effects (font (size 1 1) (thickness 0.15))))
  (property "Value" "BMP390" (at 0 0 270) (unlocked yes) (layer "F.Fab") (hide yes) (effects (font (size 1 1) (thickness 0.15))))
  (pad "1" smd rect (at -0.7874 -0.25) (size 0.254 0.2794) (layers "F.Cu" "F.Mask" "F.Paste") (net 62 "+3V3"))
  (pad "2" smd rect (at -0.7874 0.25) (size 0.254 0.2794) (layers "F.Cu" "F.Mask" "F.Paste") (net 18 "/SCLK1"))
  (pad "3" smd rect (at -0.499999 0.7874 270) (size 0.254 0.2794) (layers "F.Cu" "F.Mask" "F.Paste") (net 1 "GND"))
  (pad "4" smd rect (at 0 0.7874 270) (size 0.254 0.2794) (layers "F.Cu" "F.Mask" "F.Paste") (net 20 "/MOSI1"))
  (pad "5" smd rect (at 0.499999 0.7874 270) (size 0.254 0.2794) (layers "F.Cu" "F.Mask" "F.Paste") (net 19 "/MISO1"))
  (pad "6" smd rect (at 0.7874 0.25) (size 0.254 0.2794) (layers "F.Cu" "F.Mask" "F.Paste") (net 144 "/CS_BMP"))
  (pad "7" smd rect (at 0.7874 -0.25) (size 0.254 0.2794) (layers "F.Cu" "F.Mask" "F.Paste") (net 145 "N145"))
  (pad "8" smd rect (at 0.499999 -0.7874 270) (size 0.254 0.2794) (layers "F.Cu" "F.Mask" "F.Paste") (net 1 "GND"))
  (pad "9" smd rect (at 0 -0.7874 270) (size 0.254 0.2794) (layers "F.Cu" "F.Mask" "F.Paste") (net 1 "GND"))
  (pad "10" smd rect (at -0.499999 -0.7874 270) (size 0.254 0.2794) (layers "F.Cu" "F.Mask" "F.Paste") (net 62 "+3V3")))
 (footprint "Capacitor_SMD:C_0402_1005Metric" (layer "F.Cu") (at 144.9 108.62 -90)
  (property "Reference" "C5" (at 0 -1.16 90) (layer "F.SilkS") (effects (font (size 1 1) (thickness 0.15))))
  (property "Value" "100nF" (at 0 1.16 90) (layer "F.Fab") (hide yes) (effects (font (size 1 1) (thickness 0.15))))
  (pad "1" smd roundrect (at -0.48 0 270) (size 0.56 0.62) (layers "F.Cu" "F.Mask" "F.Paste") (roundrect_rratio 0.25) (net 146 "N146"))
  (pad "2" smd roundrect (at 0.48 0 270) (size 0.56 0.62) (layers "F.Cu" "F.Mask" "F.Paste") (roundrect_rratio 0.25) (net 1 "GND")))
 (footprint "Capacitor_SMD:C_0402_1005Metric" (layer "F.Cu") (at 143.9 108.62 90)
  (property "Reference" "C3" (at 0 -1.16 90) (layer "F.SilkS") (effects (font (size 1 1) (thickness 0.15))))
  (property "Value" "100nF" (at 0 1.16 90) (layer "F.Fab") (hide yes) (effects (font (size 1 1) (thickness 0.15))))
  (pad "1" smd roundrect (at -0.48 0 90) (size 0.56 0.62) (layers "F.Cu" "F.Mask" "F.Paste") (roundrect_rratio 0.25) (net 1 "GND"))
  (pad "2" smd roundrect (at 0.48 0 90) (size 0.56 0.62) (layers "F.Cu" "F.Mask" "F.Paste") (roundrect_rratio 0.25) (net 63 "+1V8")))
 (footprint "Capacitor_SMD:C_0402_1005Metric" (layer "F.Cu") (at 147.6 105.2 90)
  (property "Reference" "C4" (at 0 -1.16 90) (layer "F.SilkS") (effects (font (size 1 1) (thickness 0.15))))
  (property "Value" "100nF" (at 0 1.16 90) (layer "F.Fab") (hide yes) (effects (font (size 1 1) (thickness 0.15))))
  (pad "1" smd roundrect (at -0.48 0 90) (size 0.56 0.62) (layers "F.Cu" "F.Mask" "F.Paste") (roundrect_rratio 0.25) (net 62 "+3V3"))
  (pad "2" smd roundrect (at 0.48 0 90) (size 0.56 0.62) (layers "F.Cu" "F.Mask" "F.Paste") (roundrect_rratio 0.25) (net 1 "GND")))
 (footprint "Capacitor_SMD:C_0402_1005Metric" (layer "F.Cu") (at 146.9 101.4 -90)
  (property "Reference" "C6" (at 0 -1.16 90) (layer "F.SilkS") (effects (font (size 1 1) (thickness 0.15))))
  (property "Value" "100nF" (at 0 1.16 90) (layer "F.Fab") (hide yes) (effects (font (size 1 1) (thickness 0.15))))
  (pad "1" smd roundrect (at -0.48 0 270) (size 0.56 0.62) (layers "F.Cu" "F.Mask" "F.Paste") (roundrect_rratio 0.25) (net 62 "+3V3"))
  (pad "2" smd roundrect (at 0.48 0 270) (size 0.56 0.62) (layers "F.Cu" "F.Mask" "F.Paste") (roundrect_rratio 0.25) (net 1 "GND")))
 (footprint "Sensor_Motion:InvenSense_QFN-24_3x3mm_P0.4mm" (layer "F.Cu") (at 144.6 105.2)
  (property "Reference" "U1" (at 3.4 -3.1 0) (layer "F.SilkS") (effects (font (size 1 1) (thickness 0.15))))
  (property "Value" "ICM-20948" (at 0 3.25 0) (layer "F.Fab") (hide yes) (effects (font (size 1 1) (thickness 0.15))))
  (pad "1" smd roundrect (at -1.5 -1) (size 0.55 0.2) (layers "F.Cu" "F.Mask" "F.Paste") (roundrect_rratio 0.25) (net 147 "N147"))
  (pad "2" smd roundrect (at -1.5 -0.6) (size 0.55 0.2) (layers "F.Cu" "F.Mask" "F.Paste") (roundrect_rratio 0.25) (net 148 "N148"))
  (pad "3" smd roundrect (at -1.5 -0.2) (size 0.55 0.2) (layers "F.Cu" "F.Mask" "F.Paste") (roundrect_rratio 0.25) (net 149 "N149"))
  (pad "4" smd roundrect (at -1.5 0.2) (size 0.55 0.2) (layers "F.Cu" "F.Mask" "F.Paste") (roundrect_rratio 0.25) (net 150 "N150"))
  (pad "5" smd roundrect (at -1.5 0.6) (size 0.55 0.2) (layers "F.Cu" "F.Mask" "F.Paste") (roundrect_rratio 0.25) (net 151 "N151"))
  (pad "6" smd roundrect (at -1.5 1) (size 0.55 0.2) (layers "F.Cu" "F.Mask" "F.Paste") (roundrect_rratio 0.25) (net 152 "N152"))
  (pad "7" smd roundrect (at -1 1.5 90) (size 0.55 0.2) (layers "F.Cu" "F.Mask" "F.Paste") (roundrect_rratio 0.25) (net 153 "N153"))
  (pad "8" smd roundrect (at -0.6 1.5 90) (size 0.55 0.2) (layers "F.Cu" "F.Mask" "F.Paste") (roundrect_rratio 0.25) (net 63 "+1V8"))
  (pad "9" smd roundrect (at -0.2 1.5 90) (size 0.55 0.2) (layers "F.Cu" "F.Mask" "F.Paste") (roundrect_rratio 0.25) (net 19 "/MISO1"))
  (pad "10" smd roundrect (at 0.2 1.5 90) (size 0.55 0.2) (layers "F.Cu" "F.Mask" "F.Paste") (roundrect_rratio 0.25) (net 146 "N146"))
  (pad "11" smd roundrect (at 0.6 1.5 90) (size 0.55 0.2) (layers "F.Cu" "F.Mask" "F.Paste") (roundrect_rratio 0.25) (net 1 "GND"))
  (pad "12" smd roundrect (at 1 1.5 90) (size 0.55 0.2) (layers "F.Cu" "F.Mask" "F.Paste") (roundrect_rratio 0.25) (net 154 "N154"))
  (pad "13" smd roundrect (at 1.5 1) (size 0.55 0.2) (layers "F.Cu" "F.Mask" "F.Paste") (roundrect_rratio 0.25) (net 62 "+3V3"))
  (pad "14" smd roundrect (at 1.5 0.6) (size 0.55 0.2) (layers "F.Cu" "F.Mask" "F.Paste") (roundrect_rratio 0.25) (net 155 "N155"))
  (pad "15" smd roundrect (at 1.5 0.2) (size 0.55 0.2) (layers "F.Cu" "F.Mask" "F.Paste") (roundrect_rratio 0.25) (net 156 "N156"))
  (pad "16" smd roundrect (at 1.5 -0.2) (size 0.55 0.2) (layers "F.Cu" "F.Mask" "F.Paste") (roundrect_rratio 0.25) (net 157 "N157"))
  (pad "17" smd roundrect (at 1.5 -0.6) (size 0.55 0.2) (layers "F.Cu" "F.Mask" "F.Paste") (roundrect_rratio 0.25) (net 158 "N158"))
  (pad "18" smd roundrect (at 1.5 -1) (size 0.55 0.2) (layers "F.Cu" "F.Mask" "F.Paste") (roundrect_rratio 0.25) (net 1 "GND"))
  (pad "19" smd roundrect (at 1 -1.5 90) (size 0.55 0.2) (layers "F.Cu" "F.Mask" "F.Paste") (roundrect_rratio 0.25) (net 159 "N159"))
  (pad "20" smd roundrect (at 0.6 -1.5 90) (size 0.55 0.2) (layers "F.Cu" "F.Mask" "F.Paste") (roundrect_rratio 0.25) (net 1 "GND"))
  (pad "21" smd roundrect (at 0.2 -1.5 90) (size 0.55 0.2) (layers "F.Cu" "F.Mask" "F.Paste") (roundrect_rratio 0.25) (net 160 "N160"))
  (pad "22" smd roundrect (at -0.2 -1.5 90) (size 0.55 0.2) (layers "F.Cu" "F.Mask" "F.Paste") (roundrect_rratio 0.25) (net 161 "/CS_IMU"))
  (pad "23" smd roundrect (at -0.6 -1.5 90) (size 0.55 0.2) (layers "F.Cu" "F.Mask" "F.Paste") (roundrect_rratio 0.25) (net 18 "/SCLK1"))
  (pad "24" smd roundrect (at -1 -1.5 90) (size 0.55 0.2) (layers "F.Cu" "F.Mask" "F.Paste") (roundrect_rratio 0.25) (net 20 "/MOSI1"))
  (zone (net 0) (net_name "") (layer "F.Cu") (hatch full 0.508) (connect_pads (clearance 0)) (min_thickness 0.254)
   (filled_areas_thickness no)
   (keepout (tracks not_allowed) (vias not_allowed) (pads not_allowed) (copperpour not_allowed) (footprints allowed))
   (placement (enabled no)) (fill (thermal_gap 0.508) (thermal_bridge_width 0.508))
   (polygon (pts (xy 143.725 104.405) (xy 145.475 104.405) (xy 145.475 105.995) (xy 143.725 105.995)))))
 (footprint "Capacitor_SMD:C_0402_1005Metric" (layer "F.Cu") (at 145.32 99.1)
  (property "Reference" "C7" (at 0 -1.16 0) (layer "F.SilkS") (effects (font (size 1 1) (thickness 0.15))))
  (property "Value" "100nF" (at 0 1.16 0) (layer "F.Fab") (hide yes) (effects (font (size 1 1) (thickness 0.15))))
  (pad "1" smd roundrect (at -0.48 0) (size 0.56 0.62) (layers "F.Cu" "F.Mask" "F.Paste") (roundrect_rratio 0.25) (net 62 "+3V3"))
  (pad "2" smd roundrect (at 0.48 0) (size 0.56 0.62) (layers "F.Cu" "F.Mask" "F.Paste") (roundrect_rratio 0.25) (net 1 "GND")))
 (gr_circle (center 113.6 136.2) (end 115.1 136.2) (stroke (width 0.05) (type default)) (fill no) (layer "Edge.Cuts"))
 (gr_line (start 108.6 136.2) (end 108.6 74.2) (stroke (width 0.05) (type default)) (layer "Edge.Cuts"))
 (gr_circle (center 113.6 74.2) (end 113.6 72.7) (stroke (width 0.05) (type default)) (fill no) (layer "Edge.Cuts"))
 (gr_circle (center 175.6 74.2) (end 177.1 74.2) (stroke (width 0.05) (type default)) (fill no) (layer "Edge.Cuts"))
 (gr_line (start 175.6 141.2) (end 113.6 141.2) (stroke (width 0.05) (type default)) (layer "Edge.Cuts"))
 (gr_line (start 113.6 69.2) (end 175.6 69.2) (stroke (width 0.05) (type default)) (layer "Edge.Cuts"))
 (gr_line (start 180.6 74.2) (end 180.6 136.2) (stroke (width 0.05) (type default)) (layer "Edge.Cuts"))
 (gr_arc (start 180.6 136.2) (mid 179.135534 139.735534) (end 175.6 141.2) (stroke (width 0.05) (type default)) (layer "Edge.Cuts"))
 (gr_circle (center 175.6 136.2) (end 177.1 136.2) (stroke (width 0.05) (type default)) (fill no) (layer "Edge.Cuts"))
 (gr_arc (start 113.6 141.2) (mid 110.064466 139.735534) (end 108.6 136.2) (stroke (width 0.05) (type default)) (layer "Edge.Cuts"))
 (gr_arc (start 108.6 74.2) (mid 110.064466 70.664466) (end 113.6 69.2) (stroke (width 0.05) (type default)) (layer "Edge.Cuts"))
 (gr_arc (start 175.6 69.2) (mid 179.135534 70.664466) (end 180.6 74.2) (stroke (width 0.05) (type default)) (layer "Edge.Cuts"))
 (segment (start 143.9 107.5) (end 143.9 108.14) (width 0.2) (layer "F.Cu") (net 63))
 (segment (start 144 106.7) (end 144 107.4) (width 0.2) (layer "F.Cu") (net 63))
 (segment (start 144 107.4) (end 143.9 107.5) (width 0.2) (layer "F.Cu") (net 63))
 (segment (start 147.6 104.72) (end 147.08 104.2) (width 0.2) (layer "F.Cu") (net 1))
 (segment (start 145.387401 101.887399) (end 146.892601 101.887399) (width 0.2) (layer "F.Cu") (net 1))
 (segment (start 147.08 104.2) (end 146.1 104.2) (width 0.2) (layer "F.Cu") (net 1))
 (segment (start 146.892601 101.887399) (end 146.9 101.88) (width 0.2) (layer "F.Cu") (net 1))
 (segment (start 146.867401 100.887401) (end 146.9 100.92) (width 0.2) (layer "F.Cu") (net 62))
 (segment (start 144.850001 100.6) (end 144.850001 99.110001) (width 0.2) (layer "F.Cu") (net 62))
 (segment (start 145.387401 100.887401) (end 146.867401 100.887401) (width 0.2) (layer "F.Cu") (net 62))
 (segment (start 144.850001 99.110001) (end 144.84 99.1) (width 0.2) (layer "F.Cu") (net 62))
 (segment (start 147.08 106.2) (end 146.1 106.2) (width 0.2) (layer "F.Cu") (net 62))
 (segment (start 147.6 105.68) (end 147.08 106.2) (width 0.2) (layer "F.Cu") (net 62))
 (segment (start 144.9 108.14) (end 144.9 107.5) (width 0.2) (layer "F.Cu") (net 146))
 (segment (start 144.8 107.4) (end 144.8 106.7) (width 0.2) (layer "F.Cu") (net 146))
 (segment (start 144.9 107.5) (end 144.8 107.4) (width 0.2) (layer "F.Cu") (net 146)))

